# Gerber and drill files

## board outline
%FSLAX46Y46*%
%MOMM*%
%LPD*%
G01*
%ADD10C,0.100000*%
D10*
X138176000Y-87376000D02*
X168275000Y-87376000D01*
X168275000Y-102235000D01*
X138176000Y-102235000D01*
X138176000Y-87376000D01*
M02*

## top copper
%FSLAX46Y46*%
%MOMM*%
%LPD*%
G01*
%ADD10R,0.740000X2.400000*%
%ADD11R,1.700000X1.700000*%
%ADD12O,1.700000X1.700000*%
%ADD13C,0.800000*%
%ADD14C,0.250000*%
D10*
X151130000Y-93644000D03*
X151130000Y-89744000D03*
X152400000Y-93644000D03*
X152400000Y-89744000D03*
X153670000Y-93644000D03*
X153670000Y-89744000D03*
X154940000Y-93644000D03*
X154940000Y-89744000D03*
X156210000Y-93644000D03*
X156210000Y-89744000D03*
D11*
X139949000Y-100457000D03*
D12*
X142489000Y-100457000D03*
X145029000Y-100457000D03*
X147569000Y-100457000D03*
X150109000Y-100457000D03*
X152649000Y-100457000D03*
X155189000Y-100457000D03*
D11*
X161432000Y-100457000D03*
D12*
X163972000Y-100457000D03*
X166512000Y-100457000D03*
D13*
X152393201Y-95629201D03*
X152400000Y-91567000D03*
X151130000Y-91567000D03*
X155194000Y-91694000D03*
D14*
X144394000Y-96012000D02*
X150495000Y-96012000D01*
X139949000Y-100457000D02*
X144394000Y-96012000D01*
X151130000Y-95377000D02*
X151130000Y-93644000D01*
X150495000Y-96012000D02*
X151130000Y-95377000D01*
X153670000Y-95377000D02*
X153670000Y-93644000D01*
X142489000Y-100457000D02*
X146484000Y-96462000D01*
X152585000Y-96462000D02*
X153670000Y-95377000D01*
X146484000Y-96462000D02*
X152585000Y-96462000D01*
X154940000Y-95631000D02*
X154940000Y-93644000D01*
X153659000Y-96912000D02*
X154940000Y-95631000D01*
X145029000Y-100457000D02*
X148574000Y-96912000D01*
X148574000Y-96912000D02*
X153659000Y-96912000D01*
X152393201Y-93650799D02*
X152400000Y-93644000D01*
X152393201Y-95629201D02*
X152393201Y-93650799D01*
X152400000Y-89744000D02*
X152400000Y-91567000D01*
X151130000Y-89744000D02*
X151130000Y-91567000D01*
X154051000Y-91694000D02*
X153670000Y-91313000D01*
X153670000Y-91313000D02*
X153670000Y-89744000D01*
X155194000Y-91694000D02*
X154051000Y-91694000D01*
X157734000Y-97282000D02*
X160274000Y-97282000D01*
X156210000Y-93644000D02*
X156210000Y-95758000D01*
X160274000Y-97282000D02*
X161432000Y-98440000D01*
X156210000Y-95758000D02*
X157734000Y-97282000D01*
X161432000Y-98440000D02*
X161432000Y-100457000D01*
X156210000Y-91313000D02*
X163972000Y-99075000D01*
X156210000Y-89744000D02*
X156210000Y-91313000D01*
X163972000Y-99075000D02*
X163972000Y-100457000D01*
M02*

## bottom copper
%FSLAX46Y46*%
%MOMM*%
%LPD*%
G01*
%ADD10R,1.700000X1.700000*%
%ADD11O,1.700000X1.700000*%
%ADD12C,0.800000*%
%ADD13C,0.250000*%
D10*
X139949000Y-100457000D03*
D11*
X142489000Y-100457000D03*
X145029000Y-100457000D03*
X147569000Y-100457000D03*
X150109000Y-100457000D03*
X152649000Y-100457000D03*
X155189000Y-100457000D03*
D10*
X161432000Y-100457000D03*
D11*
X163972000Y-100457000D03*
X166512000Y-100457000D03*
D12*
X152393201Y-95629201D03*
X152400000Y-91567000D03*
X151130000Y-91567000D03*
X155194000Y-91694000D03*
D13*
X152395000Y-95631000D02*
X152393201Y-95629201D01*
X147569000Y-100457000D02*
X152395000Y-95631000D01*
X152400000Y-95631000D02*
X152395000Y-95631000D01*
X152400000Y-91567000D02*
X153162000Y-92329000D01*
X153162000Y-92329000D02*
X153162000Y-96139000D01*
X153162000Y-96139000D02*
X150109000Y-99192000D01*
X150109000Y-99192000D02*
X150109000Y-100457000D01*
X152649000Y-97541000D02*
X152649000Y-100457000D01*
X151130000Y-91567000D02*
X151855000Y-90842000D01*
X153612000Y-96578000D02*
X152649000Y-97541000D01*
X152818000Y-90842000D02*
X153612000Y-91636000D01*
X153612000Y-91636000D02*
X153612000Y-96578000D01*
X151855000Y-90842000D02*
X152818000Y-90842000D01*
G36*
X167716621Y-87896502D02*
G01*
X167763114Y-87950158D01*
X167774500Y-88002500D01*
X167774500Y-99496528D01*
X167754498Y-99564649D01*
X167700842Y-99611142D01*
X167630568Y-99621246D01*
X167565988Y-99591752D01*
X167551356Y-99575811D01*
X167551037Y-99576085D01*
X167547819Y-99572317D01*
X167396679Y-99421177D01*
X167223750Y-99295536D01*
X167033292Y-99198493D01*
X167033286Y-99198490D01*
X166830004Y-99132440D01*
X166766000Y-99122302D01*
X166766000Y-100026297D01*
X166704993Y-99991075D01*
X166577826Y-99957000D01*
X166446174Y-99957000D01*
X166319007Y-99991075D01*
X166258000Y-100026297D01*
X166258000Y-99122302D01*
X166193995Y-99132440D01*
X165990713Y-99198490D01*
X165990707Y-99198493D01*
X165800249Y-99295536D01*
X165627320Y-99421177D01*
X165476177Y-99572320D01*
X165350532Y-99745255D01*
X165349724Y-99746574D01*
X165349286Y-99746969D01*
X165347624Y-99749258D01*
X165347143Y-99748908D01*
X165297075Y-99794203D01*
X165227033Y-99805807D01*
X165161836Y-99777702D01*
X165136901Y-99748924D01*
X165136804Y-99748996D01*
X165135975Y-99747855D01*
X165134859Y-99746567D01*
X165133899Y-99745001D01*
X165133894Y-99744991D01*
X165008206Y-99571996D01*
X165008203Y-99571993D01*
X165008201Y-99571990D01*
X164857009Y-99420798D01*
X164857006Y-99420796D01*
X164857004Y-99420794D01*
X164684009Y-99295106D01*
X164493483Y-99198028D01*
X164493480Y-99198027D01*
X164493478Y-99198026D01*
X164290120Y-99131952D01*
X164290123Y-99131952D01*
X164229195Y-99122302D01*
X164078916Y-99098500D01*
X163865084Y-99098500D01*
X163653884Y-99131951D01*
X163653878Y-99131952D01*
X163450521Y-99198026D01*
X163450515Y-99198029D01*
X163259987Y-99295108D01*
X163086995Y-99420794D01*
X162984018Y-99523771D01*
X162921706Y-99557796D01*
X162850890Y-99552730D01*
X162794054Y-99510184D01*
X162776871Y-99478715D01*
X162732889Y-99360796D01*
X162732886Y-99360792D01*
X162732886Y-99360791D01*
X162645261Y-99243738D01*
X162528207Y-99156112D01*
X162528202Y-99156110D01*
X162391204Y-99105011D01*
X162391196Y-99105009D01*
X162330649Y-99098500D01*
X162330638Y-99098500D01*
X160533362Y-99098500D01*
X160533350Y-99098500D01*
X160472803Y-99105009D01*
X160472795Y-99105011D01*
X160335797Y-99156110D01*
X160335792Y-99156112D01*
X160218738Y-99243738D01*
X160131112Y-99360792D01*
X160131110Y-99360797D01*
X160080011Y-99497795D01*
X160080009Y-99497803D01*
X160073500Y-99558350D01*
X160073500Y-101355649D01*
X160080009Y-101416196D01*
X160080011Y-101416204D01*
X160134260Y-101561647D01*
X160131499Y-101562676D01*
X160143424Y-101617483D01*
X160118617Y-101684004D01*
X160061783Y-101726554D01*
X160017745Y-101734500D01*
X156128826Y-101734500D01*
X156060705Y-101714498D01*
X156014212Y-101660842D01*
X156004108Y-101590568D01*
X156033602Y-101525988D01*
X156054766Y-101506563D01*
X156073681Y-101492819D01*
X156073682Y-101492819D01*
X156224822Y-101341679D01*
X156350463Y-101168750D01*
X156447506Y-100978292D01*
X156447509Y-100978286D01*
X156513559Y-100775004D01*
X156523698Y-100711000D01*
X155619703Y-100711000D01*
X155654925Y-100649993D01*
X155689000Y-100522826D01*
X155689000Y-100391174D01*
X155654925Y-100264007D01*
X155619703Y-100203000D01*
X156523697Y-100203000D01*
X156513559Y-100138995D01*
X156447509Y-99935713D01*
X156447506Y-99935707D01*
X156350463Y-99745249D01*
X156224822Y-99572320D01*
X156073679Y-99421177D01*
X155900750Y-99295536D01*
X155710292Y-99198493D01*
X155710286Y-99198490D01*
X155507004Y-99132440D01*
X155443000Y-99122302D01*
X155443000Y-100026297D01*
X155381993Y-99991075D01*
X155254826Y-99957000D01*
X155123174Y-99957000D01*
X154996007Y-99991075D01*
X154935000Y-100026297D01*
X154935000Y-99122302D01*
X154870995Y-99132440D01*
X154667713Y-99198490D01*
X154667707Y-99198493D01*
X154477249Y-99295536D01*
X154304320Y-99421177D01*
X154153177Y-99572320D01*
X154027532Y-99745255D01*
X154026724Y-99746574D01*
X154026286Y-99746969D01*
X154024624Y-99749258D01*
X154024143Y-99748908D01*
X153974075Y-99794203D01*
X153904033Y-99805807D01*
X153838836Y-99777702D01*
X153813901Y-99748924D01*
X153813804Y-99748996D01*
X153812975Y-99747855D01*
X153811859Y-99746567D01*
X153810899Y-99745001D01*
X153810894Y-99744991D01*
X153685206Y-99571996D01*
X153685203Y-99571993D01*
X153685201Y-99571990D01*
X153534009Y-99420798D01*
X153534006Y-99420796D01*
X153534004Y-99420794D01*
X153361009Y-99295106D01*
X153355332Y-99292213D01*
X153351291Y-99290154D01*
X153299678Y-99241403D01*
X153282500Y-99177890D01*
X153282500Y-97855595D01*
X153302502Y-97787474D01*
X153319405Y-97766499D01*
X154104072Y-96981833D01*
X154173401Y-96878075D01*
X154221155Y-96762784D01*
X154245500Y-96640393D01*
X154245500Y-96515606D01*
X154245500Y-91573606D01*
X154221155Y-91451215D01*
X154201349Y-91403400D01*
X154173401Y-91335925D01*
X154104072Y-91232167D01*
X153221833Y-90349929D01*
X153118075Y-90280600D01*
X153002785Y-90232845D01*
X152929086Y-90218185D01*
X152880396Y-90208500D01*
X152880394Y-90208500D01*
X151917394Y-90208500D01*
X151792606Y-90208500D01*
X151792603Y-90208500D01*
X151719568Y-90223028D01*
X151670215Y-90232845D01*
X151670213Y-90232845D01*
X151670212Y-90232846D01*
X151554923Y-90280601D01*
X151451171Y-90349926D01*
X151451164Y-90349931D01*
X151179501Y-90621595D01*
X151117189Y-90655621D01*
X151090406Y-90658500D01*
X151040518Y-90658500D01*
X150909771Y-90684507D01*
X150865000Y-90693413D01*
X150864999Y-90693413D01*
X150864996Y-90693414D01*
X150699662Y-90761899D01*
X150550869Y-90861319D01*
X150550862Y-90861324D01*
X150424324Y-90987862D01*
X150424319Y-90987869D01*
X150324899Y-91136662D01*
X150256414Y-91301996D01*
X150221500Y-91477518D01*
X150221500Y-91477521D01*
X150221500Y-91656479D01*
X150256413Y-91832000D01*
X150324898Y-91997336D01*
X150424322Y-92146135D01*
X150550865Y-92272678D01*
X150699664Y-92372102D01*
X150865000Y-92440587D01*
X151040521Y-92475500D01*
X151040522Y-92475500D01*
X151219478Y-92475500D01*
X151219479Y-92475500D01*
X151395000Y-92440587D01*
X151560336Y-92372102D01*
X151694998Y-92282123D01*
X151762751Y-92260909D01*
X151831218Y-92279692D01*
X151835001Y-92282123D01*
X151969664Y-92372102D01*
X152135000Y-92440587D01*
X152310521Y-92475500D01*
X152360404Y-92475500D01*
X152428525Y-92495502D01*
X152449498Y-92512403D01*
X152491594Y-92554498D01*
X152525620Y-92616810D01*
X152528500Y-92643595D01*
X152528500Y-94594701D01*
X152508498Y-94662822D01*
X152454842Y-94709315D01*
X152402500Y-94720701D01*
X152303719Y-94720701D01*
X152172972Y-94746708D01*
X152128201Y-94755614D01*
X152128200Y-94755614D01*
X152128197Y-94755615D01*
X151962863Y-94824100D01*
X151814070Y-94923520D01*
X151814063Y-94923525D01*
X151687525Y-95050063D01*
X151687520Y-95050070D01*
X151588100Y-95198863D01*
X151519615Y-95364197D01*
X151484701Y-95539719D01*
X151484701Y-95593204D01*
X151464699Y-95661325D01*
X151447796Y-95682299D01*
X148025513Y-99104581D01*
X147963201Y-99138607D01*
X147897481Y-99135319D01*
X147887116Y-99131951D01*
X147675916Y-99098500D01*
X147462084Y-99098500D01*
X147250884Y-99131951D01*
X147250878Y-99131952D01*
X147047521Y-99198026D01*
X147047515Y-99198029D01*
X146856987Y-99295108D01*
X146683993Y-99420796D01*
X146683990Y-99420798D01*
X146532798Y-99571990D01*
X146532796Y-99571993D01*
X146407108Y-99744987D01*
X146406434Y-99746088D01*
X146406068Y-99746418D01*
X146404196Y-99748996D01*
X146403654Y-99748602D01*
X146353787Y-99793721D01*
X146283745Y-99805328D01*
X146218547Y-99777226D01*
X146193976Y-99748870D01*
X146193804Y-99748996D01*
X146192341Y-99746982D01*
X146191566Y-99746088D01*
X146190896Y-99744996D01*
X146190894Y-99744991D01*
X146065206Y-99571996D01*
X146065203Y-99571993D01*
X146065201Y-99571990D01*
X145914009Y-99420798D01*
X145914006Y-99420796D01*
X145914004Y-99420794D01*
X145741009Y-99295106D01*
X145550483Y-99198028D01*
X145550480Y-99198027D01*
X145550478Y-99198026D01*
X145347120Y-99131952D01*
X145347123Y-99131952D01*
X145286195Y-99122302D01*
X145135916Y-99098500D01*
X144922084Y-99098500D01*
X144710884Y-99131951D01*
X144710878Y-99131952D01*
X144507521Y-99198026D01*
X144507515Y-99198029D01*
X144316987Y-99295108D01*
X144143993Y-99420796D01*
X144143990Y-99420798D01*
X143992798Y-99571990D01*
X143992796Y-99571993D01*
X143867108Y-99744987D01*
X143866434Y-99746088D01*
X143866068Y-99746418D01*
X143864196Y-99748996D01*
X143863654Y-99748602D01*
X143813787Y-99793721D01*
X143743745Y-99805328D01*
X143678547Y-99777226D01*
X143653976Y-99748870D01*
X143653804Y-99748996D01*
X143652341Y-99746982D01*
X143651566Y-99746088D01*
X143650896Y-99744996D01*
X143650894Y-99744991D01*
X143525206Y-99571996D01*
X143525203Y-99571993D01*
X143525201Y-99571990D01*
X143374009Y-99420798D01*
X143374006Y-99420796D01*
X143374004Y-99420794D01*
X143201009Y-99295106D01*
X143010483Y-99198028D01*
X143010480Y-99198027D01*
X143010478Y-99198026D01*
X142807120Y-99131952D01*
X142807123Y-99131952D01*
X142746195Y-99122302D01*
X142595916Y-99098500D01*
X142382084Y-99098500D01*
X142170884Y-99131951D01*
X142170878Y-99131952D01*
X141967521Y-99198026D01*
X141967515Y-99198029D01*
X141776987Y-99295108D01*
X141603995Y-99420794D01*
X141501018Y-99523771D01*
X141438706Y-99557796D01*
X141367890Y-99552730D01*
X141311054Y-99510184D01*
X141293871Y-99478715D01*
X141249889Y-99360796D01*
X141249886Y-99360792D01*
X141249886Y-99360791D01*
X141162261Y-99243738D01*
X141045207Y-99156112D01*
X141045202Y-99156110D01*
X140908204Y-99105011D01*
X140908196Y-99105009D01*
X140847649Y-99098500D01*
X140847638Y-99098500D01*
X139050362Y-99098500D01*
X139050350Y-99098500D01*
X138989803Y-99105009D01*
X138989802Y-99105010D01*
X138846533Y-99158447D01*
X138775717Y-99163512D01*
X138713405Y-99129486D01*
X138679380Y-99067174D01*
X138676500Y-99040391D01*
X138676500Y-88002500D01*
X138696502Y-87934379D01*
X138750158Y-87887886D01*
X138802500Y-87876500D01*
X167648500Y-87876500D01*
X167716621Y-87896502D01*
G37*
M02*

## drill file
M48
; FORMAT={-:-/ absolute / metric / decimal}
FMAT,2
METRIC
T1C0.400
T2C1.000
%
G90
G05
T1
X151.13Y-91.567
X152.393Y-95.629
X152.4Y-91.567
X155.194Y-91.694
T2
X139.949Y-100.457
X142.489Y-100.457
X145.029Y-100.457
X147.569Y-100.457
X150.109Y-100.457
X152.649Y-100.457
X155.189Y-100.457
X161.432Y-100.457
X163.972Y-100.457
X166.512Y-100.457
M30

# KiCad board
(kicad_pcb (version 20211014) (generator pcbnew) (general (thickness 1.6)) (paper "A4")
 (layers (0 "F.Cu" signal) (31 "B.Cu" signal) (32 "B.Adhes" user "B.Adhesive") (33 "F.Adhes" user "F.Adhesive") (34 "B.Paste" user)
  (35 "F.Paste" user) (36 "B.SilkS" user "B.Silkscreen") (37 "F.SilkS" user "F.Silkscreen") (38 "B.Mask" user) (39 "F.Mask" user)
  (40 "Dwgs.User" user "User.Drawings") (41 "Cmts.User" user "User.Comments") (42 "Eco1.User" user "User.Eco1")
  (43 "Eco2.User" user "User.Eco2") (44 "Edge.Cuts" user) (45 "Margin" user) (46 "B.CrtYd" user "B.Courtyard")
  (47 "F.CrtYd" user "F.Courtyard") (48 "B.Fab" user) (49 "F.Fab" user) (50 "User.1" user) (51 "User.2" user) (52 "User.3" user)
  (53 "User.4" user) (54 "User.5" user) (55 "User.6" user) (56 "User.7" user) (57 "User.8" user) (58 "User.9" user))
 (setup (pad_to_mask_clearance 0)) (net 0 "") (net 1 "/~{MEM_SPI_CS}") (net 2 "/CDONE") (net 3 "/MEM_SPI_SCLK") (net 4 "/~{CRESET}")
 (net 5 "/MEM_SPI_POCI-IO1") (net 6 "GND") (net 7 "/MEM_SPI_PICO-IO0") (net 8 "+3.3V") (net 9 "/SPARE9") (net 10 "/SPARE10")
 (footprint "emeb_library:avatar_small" (layer "F.Cu") (at 164.415172 93.026757)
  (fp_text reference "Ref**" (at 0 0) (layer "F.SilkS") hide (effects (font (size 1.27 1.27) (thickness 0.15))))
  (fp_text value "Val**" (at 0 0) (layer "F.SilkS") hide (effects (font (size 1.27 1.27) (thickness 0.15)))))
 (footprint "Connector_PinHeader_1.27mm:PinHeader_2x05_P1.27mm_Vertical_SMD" (layer "F.Cu") (at 153.67 91.694 90)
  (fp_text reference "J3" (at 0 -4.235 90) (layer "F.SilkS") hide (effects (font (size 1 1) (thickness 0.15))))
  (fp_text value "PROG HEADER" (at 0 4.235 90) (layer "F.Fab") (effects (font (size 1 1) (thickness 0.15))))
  (pad "1" smd rect (at -1.95 -2.54 90) (size 2.4 0.74) (layers "F.Cu" "F.Paste" "F.Mask") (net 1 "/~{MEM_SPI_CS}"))
  (pad "2" smd rect (at 1.95 -2.54 90) (size 2.4 0.74) (layers "F.Cu" "F.Paste" "F.Mask") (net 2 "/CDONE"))
  (pad "3" smd rect (at -1.95 -1.27 90) (size 2.4 0.74) (layers "F.Cu" "F.Paste" "F.Mask") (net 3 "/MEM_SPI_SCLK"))
  (pad "4" smd rect (at 1.95 -1.27 90) (size 2.4 0.74) (layers "F.Cu" "F.Paste" "F.Mask") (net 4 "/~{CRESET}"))
  (pad "5" smd rect (at -1.95 0 90) (size 2.4 0.74) (layers "F.Cu" "F.Paste" "F.Mask") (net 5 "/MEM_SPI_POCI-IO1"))
  (pad "6" smd rect (at 1.95 0 90) (size 2.4 0.74) (layers "F.Cu" "F.Paste" "F.Mask") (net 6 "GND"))
  (pad "7" smd rect (at -1.95 1.27 90) (size 2.4 0.74) (layers "F.Cu" "F.Paste" "F.Mask") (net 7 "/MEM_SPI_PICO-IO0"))
  (pad "8" smd rect (at 1.95 1.27 90) (size 2.4 0.74) (layers "F.Cu" "F.Paste" "F.Mask") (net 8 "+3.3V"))
  (pad "9" smd rect (at -1.95 2.54 90) (size 2.4 0.74) (layers "F.Cu" "F.Paste" "F.Mask") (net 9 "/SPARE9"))
  (pad "10" smd rect (at 1.95 2.54 90) (size 2.4 0.74) (layers "F.Cu" "F.Paste" "F.Mask") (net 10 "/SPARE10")))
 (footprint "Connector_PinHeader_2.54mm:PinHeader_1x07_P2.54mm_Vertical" (layer "F.Cu") (at 139.949 100.457 90)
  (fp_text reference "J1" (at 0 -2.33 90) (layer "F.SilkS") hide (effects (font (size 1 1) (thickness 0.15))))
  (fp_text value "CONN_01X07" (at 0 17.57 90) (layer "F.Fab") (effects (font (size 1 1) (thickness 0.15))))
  (pad "1" thru_hole rect (at 0 0 90) (size 1.7 1.7) (drill 1) (layers *.Cu *.Mask) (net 1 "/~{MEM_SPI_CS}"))
  (pad "2" thru_hole oval (at 0 2.54 90) (size 1.7 1.7) (drill 1) (layers *.Cu *.Mask) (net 5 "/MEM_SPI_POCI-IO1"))
  (pad "3" thru_hole oval (at 0 5.08 90) (size 1.7 1.7) (drill 1) (layers *.Cu *.Mask) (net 7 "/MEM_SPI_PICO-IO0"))
  (pad "4" thru_hole oval (at 0 7.62 90) (size 1.7 1.7) (drill 1) (layers *.Cu *.Mask) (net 3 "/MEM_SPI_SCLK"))
  (pad "5" thru_hole oval (at 0 10.16 90) (size 1.7 1.7) (drill 1) (layers *.Cu *.Mask) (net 4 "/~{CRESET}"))
  (pad "6" thru_hole oval (at 0 12.7 90) (size 1.7 1.7) (drill 1) (layers *.Cu *.Mask) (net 2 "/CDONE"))
  (pad "7" thru_hole oval (at 0 15.24 90) (size 1.7 1.7) (drill 1) (layers *.Cu *.Mask) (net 6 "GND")))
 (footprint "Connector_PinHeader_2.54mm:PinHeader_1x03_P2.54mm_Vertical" (layer "F.Cu") (at 161.432 100.457 90)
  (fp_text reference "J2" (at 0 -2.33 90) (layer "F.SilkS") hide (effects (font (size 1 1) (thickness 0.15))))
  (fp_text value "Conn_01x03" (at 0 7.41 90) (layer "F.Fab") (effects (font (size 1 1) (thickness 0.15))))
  (pad "1" thru_hole rect (at 0 0 90) (size 1.7 1.7) (drill 1) (layers *.Cu *.Mask) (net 9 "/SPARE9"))
  (pad "2" thru_hole oval (at 0 2.54 90) (size 1.7 1.7) (drill 1) (layers *.Cu *.Mask) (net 10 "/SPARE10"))
  (pad "3" thru_hole oval (at 0 5.08 90) (size 1.7 1.7) (drill 1) (layers *.Cu *.Mask) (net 6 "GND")))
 (gr_rect (start 138.176 102.235) (end 168.275 87.376) (layer "Edge.Cuts") (width 0.1) (fill none))
 (segment (start 144.394 96.012) (end 150.495 96.012) (width 0.25) (layer "F.Cu") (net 1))
 (segment (start 139.949 100.457) (end 144.394 96.012) (width 0.25) (layer "F.Cu") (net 1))
 (segment (start 151.13 95.377) (end 151.13 93.644) (width 0.25) (layer "F.Cu") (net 1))
 (segment (start 150.495 96.012) (end 151.13 95.377) (width 0.25) (layer "F.Cu") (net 1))
 (segment (start 153.67 95.377) (end 153.67 93.644) (width 0.25) (layer "F.Cu") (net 5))
 (segment (start 142.489 100.457) (end 146.484 96.462) (width 0.25) (layer "F.Cu") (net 5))
 (segment (start 152.585 96.462) (end 153.67 95.377) (width 0.25) (layer "F.Cu") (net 5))
 (segment (start 146.484 96.462) (end 152.585 96.462) (width 0.25) (layer "F.Cu") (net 5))
 (segment (start 154.94 95.631) (end 154.94 93.644) (width 0.25) (layer "F.Cu") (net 7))
 (segment (start 153.659 96.912) (end 154.94 95.631) (width 0.25) (layer "F.Cu") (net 7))
 (segment (start 145.029 100.457) (end 148.574 96.912) (width 0.25) (layer "F.Cu") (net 7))
 (segment (start 148.574 96.912) (end 153.659 96.912) (width 0.25) (layer "F.Cu") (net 7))
 (segment (start 152.393201 93.650799) (end 152.4 93.644) (width 0.25) (layer "F.Cu") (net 3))
 (segment (start 152.393201 95.629201) (end 152.393201 93.650799) (width 0.25) (layer "F.Cu") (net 3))
 (via (at 152.393201 95.629201) (size 0.8) (drill 0.4) (layers "F.Cu" "B.Cu") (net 3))
 (segment (start 152.395 95.631) (end 152.393201 95.629201) (width 0.25) (layer "B.Cu") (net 3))
 (segment (start 147.569 100.457) (end 152.395 95.631) (width 0.25) (layer "B.Cu") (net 3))
 (segment (start 152.4 95.631) (end 152.395 95.631) (width 0.25) (layer "B.Cu") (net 3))
 (segment (start 152.4 89.744) (end 152.4 91.567) (width 0.25) (layer "F.Cu") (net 4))
 (via (at 152.4 91.567) (size 0.8) (drill 0.4) (layers "F.Cu" "B.Cu") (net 4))
 (segment (start 152.4 91.567) (end 153.162 92.329) (width 0.25) (layer "B.Cu") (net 4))
 (segment (start 153.162 92.329) (end 153.162 96.139) (width 0.25) (layer "B.Cu") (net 4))
 (segment (start 153.162 96.139) (end 150.109 99.192) (width 0.25) (layer "B.Cu") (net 4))
 (segment (start 150.109 99.192) (end 150.109 100.457) (width 0.25) (layer "B.Cu") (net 4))
 (segment (start 151.13 89.744) (end 151.13 91.567) (width 0.25) (layer "F.Cu") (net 2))
 (via (at 151.13 91.567) (size 0.8) (drill 0.4) (layers "F.Cu" "B.Cu") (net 2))
 (segment (start 152.649 97.541) (end 152.649 100.457) (width 0.25) (layer "B.Cu") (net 2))
 (segment (start 151.13 91.567) (end 151.855 90.842) (width 0.25) (layer "B.Cu") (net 2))
 (segment (start 153.612 96.578) (end 152.649 97.541) (width 0.25) (layer "B.Cu") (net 2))
 (segment (start 152.818 90.842) (end 153.612 91.636) (width 0.25) (layer "B.Cu") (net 2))
 (segment (start 153.612 91.636) (end 153.612 96.578) (width 0.25) (layer "B.Cu") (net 2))
 (segment (start 151.855 90.842) (end 152.818 90.842) (width 0.25) (layer "B.Cu") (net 2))
 (segment (start 154.051 91.694) (end 153.67 91.313) (width 0.25) (layer "F.Cu") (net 6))
 (segment (start 153.67 91.313) (end 153.67 89.744) (width 0.25) (layer "F.Cu") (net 6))
 (segment (start 155.194 91.694) (end 154.051 91.694) (width 0.25) (layer "F.Cu") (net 6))
 (via (at 155.194 91.694) (size 0.8) (drill 0.4) (layers "F.Cu" "B.Cu") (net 6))
 (segment (start 157.734 97.282) (end 160.274 97.282) (width 0.25) (layer "F.Cu") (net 9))
 (segment (start 156.21 93.644) (end 156.21 95.758) (width 0.25) (layer "F.Cu") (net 9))
 (segment (start 160.274 97.282) (end 161.432 98.44) (width 0.25) (layer "F.Cu") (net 9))
 (segment (start 156.21 95.758) (end 157.734 97.282) (width 0.25) (layer "F.Cu") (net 9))
 (segment (start 161.432 98.44) (end 161.432 100.457) (width 0.25) (layer "F.Cu") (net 9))
 (segment (start 156.21 91.313) (end 163.972 99.075) (width 0.25) (layer "F.Cu") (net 10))
 (segment (start 156.21 89.744) (end 156.21 91.313) (width 0.25) (layer "F.Cu") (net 10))
 (segment (start 163.972 99.075) (end 163.972 100.457) (width 0.25) (layer "F.Cu") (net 10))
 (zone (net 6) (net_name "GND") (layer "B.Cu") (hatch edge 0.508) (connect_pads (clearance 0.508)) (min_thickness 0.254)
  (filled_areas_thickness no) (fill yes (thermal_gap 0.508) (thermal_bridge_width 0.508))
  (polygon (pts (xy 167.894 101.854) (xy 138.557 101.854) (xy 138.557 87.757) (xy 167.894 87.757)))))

